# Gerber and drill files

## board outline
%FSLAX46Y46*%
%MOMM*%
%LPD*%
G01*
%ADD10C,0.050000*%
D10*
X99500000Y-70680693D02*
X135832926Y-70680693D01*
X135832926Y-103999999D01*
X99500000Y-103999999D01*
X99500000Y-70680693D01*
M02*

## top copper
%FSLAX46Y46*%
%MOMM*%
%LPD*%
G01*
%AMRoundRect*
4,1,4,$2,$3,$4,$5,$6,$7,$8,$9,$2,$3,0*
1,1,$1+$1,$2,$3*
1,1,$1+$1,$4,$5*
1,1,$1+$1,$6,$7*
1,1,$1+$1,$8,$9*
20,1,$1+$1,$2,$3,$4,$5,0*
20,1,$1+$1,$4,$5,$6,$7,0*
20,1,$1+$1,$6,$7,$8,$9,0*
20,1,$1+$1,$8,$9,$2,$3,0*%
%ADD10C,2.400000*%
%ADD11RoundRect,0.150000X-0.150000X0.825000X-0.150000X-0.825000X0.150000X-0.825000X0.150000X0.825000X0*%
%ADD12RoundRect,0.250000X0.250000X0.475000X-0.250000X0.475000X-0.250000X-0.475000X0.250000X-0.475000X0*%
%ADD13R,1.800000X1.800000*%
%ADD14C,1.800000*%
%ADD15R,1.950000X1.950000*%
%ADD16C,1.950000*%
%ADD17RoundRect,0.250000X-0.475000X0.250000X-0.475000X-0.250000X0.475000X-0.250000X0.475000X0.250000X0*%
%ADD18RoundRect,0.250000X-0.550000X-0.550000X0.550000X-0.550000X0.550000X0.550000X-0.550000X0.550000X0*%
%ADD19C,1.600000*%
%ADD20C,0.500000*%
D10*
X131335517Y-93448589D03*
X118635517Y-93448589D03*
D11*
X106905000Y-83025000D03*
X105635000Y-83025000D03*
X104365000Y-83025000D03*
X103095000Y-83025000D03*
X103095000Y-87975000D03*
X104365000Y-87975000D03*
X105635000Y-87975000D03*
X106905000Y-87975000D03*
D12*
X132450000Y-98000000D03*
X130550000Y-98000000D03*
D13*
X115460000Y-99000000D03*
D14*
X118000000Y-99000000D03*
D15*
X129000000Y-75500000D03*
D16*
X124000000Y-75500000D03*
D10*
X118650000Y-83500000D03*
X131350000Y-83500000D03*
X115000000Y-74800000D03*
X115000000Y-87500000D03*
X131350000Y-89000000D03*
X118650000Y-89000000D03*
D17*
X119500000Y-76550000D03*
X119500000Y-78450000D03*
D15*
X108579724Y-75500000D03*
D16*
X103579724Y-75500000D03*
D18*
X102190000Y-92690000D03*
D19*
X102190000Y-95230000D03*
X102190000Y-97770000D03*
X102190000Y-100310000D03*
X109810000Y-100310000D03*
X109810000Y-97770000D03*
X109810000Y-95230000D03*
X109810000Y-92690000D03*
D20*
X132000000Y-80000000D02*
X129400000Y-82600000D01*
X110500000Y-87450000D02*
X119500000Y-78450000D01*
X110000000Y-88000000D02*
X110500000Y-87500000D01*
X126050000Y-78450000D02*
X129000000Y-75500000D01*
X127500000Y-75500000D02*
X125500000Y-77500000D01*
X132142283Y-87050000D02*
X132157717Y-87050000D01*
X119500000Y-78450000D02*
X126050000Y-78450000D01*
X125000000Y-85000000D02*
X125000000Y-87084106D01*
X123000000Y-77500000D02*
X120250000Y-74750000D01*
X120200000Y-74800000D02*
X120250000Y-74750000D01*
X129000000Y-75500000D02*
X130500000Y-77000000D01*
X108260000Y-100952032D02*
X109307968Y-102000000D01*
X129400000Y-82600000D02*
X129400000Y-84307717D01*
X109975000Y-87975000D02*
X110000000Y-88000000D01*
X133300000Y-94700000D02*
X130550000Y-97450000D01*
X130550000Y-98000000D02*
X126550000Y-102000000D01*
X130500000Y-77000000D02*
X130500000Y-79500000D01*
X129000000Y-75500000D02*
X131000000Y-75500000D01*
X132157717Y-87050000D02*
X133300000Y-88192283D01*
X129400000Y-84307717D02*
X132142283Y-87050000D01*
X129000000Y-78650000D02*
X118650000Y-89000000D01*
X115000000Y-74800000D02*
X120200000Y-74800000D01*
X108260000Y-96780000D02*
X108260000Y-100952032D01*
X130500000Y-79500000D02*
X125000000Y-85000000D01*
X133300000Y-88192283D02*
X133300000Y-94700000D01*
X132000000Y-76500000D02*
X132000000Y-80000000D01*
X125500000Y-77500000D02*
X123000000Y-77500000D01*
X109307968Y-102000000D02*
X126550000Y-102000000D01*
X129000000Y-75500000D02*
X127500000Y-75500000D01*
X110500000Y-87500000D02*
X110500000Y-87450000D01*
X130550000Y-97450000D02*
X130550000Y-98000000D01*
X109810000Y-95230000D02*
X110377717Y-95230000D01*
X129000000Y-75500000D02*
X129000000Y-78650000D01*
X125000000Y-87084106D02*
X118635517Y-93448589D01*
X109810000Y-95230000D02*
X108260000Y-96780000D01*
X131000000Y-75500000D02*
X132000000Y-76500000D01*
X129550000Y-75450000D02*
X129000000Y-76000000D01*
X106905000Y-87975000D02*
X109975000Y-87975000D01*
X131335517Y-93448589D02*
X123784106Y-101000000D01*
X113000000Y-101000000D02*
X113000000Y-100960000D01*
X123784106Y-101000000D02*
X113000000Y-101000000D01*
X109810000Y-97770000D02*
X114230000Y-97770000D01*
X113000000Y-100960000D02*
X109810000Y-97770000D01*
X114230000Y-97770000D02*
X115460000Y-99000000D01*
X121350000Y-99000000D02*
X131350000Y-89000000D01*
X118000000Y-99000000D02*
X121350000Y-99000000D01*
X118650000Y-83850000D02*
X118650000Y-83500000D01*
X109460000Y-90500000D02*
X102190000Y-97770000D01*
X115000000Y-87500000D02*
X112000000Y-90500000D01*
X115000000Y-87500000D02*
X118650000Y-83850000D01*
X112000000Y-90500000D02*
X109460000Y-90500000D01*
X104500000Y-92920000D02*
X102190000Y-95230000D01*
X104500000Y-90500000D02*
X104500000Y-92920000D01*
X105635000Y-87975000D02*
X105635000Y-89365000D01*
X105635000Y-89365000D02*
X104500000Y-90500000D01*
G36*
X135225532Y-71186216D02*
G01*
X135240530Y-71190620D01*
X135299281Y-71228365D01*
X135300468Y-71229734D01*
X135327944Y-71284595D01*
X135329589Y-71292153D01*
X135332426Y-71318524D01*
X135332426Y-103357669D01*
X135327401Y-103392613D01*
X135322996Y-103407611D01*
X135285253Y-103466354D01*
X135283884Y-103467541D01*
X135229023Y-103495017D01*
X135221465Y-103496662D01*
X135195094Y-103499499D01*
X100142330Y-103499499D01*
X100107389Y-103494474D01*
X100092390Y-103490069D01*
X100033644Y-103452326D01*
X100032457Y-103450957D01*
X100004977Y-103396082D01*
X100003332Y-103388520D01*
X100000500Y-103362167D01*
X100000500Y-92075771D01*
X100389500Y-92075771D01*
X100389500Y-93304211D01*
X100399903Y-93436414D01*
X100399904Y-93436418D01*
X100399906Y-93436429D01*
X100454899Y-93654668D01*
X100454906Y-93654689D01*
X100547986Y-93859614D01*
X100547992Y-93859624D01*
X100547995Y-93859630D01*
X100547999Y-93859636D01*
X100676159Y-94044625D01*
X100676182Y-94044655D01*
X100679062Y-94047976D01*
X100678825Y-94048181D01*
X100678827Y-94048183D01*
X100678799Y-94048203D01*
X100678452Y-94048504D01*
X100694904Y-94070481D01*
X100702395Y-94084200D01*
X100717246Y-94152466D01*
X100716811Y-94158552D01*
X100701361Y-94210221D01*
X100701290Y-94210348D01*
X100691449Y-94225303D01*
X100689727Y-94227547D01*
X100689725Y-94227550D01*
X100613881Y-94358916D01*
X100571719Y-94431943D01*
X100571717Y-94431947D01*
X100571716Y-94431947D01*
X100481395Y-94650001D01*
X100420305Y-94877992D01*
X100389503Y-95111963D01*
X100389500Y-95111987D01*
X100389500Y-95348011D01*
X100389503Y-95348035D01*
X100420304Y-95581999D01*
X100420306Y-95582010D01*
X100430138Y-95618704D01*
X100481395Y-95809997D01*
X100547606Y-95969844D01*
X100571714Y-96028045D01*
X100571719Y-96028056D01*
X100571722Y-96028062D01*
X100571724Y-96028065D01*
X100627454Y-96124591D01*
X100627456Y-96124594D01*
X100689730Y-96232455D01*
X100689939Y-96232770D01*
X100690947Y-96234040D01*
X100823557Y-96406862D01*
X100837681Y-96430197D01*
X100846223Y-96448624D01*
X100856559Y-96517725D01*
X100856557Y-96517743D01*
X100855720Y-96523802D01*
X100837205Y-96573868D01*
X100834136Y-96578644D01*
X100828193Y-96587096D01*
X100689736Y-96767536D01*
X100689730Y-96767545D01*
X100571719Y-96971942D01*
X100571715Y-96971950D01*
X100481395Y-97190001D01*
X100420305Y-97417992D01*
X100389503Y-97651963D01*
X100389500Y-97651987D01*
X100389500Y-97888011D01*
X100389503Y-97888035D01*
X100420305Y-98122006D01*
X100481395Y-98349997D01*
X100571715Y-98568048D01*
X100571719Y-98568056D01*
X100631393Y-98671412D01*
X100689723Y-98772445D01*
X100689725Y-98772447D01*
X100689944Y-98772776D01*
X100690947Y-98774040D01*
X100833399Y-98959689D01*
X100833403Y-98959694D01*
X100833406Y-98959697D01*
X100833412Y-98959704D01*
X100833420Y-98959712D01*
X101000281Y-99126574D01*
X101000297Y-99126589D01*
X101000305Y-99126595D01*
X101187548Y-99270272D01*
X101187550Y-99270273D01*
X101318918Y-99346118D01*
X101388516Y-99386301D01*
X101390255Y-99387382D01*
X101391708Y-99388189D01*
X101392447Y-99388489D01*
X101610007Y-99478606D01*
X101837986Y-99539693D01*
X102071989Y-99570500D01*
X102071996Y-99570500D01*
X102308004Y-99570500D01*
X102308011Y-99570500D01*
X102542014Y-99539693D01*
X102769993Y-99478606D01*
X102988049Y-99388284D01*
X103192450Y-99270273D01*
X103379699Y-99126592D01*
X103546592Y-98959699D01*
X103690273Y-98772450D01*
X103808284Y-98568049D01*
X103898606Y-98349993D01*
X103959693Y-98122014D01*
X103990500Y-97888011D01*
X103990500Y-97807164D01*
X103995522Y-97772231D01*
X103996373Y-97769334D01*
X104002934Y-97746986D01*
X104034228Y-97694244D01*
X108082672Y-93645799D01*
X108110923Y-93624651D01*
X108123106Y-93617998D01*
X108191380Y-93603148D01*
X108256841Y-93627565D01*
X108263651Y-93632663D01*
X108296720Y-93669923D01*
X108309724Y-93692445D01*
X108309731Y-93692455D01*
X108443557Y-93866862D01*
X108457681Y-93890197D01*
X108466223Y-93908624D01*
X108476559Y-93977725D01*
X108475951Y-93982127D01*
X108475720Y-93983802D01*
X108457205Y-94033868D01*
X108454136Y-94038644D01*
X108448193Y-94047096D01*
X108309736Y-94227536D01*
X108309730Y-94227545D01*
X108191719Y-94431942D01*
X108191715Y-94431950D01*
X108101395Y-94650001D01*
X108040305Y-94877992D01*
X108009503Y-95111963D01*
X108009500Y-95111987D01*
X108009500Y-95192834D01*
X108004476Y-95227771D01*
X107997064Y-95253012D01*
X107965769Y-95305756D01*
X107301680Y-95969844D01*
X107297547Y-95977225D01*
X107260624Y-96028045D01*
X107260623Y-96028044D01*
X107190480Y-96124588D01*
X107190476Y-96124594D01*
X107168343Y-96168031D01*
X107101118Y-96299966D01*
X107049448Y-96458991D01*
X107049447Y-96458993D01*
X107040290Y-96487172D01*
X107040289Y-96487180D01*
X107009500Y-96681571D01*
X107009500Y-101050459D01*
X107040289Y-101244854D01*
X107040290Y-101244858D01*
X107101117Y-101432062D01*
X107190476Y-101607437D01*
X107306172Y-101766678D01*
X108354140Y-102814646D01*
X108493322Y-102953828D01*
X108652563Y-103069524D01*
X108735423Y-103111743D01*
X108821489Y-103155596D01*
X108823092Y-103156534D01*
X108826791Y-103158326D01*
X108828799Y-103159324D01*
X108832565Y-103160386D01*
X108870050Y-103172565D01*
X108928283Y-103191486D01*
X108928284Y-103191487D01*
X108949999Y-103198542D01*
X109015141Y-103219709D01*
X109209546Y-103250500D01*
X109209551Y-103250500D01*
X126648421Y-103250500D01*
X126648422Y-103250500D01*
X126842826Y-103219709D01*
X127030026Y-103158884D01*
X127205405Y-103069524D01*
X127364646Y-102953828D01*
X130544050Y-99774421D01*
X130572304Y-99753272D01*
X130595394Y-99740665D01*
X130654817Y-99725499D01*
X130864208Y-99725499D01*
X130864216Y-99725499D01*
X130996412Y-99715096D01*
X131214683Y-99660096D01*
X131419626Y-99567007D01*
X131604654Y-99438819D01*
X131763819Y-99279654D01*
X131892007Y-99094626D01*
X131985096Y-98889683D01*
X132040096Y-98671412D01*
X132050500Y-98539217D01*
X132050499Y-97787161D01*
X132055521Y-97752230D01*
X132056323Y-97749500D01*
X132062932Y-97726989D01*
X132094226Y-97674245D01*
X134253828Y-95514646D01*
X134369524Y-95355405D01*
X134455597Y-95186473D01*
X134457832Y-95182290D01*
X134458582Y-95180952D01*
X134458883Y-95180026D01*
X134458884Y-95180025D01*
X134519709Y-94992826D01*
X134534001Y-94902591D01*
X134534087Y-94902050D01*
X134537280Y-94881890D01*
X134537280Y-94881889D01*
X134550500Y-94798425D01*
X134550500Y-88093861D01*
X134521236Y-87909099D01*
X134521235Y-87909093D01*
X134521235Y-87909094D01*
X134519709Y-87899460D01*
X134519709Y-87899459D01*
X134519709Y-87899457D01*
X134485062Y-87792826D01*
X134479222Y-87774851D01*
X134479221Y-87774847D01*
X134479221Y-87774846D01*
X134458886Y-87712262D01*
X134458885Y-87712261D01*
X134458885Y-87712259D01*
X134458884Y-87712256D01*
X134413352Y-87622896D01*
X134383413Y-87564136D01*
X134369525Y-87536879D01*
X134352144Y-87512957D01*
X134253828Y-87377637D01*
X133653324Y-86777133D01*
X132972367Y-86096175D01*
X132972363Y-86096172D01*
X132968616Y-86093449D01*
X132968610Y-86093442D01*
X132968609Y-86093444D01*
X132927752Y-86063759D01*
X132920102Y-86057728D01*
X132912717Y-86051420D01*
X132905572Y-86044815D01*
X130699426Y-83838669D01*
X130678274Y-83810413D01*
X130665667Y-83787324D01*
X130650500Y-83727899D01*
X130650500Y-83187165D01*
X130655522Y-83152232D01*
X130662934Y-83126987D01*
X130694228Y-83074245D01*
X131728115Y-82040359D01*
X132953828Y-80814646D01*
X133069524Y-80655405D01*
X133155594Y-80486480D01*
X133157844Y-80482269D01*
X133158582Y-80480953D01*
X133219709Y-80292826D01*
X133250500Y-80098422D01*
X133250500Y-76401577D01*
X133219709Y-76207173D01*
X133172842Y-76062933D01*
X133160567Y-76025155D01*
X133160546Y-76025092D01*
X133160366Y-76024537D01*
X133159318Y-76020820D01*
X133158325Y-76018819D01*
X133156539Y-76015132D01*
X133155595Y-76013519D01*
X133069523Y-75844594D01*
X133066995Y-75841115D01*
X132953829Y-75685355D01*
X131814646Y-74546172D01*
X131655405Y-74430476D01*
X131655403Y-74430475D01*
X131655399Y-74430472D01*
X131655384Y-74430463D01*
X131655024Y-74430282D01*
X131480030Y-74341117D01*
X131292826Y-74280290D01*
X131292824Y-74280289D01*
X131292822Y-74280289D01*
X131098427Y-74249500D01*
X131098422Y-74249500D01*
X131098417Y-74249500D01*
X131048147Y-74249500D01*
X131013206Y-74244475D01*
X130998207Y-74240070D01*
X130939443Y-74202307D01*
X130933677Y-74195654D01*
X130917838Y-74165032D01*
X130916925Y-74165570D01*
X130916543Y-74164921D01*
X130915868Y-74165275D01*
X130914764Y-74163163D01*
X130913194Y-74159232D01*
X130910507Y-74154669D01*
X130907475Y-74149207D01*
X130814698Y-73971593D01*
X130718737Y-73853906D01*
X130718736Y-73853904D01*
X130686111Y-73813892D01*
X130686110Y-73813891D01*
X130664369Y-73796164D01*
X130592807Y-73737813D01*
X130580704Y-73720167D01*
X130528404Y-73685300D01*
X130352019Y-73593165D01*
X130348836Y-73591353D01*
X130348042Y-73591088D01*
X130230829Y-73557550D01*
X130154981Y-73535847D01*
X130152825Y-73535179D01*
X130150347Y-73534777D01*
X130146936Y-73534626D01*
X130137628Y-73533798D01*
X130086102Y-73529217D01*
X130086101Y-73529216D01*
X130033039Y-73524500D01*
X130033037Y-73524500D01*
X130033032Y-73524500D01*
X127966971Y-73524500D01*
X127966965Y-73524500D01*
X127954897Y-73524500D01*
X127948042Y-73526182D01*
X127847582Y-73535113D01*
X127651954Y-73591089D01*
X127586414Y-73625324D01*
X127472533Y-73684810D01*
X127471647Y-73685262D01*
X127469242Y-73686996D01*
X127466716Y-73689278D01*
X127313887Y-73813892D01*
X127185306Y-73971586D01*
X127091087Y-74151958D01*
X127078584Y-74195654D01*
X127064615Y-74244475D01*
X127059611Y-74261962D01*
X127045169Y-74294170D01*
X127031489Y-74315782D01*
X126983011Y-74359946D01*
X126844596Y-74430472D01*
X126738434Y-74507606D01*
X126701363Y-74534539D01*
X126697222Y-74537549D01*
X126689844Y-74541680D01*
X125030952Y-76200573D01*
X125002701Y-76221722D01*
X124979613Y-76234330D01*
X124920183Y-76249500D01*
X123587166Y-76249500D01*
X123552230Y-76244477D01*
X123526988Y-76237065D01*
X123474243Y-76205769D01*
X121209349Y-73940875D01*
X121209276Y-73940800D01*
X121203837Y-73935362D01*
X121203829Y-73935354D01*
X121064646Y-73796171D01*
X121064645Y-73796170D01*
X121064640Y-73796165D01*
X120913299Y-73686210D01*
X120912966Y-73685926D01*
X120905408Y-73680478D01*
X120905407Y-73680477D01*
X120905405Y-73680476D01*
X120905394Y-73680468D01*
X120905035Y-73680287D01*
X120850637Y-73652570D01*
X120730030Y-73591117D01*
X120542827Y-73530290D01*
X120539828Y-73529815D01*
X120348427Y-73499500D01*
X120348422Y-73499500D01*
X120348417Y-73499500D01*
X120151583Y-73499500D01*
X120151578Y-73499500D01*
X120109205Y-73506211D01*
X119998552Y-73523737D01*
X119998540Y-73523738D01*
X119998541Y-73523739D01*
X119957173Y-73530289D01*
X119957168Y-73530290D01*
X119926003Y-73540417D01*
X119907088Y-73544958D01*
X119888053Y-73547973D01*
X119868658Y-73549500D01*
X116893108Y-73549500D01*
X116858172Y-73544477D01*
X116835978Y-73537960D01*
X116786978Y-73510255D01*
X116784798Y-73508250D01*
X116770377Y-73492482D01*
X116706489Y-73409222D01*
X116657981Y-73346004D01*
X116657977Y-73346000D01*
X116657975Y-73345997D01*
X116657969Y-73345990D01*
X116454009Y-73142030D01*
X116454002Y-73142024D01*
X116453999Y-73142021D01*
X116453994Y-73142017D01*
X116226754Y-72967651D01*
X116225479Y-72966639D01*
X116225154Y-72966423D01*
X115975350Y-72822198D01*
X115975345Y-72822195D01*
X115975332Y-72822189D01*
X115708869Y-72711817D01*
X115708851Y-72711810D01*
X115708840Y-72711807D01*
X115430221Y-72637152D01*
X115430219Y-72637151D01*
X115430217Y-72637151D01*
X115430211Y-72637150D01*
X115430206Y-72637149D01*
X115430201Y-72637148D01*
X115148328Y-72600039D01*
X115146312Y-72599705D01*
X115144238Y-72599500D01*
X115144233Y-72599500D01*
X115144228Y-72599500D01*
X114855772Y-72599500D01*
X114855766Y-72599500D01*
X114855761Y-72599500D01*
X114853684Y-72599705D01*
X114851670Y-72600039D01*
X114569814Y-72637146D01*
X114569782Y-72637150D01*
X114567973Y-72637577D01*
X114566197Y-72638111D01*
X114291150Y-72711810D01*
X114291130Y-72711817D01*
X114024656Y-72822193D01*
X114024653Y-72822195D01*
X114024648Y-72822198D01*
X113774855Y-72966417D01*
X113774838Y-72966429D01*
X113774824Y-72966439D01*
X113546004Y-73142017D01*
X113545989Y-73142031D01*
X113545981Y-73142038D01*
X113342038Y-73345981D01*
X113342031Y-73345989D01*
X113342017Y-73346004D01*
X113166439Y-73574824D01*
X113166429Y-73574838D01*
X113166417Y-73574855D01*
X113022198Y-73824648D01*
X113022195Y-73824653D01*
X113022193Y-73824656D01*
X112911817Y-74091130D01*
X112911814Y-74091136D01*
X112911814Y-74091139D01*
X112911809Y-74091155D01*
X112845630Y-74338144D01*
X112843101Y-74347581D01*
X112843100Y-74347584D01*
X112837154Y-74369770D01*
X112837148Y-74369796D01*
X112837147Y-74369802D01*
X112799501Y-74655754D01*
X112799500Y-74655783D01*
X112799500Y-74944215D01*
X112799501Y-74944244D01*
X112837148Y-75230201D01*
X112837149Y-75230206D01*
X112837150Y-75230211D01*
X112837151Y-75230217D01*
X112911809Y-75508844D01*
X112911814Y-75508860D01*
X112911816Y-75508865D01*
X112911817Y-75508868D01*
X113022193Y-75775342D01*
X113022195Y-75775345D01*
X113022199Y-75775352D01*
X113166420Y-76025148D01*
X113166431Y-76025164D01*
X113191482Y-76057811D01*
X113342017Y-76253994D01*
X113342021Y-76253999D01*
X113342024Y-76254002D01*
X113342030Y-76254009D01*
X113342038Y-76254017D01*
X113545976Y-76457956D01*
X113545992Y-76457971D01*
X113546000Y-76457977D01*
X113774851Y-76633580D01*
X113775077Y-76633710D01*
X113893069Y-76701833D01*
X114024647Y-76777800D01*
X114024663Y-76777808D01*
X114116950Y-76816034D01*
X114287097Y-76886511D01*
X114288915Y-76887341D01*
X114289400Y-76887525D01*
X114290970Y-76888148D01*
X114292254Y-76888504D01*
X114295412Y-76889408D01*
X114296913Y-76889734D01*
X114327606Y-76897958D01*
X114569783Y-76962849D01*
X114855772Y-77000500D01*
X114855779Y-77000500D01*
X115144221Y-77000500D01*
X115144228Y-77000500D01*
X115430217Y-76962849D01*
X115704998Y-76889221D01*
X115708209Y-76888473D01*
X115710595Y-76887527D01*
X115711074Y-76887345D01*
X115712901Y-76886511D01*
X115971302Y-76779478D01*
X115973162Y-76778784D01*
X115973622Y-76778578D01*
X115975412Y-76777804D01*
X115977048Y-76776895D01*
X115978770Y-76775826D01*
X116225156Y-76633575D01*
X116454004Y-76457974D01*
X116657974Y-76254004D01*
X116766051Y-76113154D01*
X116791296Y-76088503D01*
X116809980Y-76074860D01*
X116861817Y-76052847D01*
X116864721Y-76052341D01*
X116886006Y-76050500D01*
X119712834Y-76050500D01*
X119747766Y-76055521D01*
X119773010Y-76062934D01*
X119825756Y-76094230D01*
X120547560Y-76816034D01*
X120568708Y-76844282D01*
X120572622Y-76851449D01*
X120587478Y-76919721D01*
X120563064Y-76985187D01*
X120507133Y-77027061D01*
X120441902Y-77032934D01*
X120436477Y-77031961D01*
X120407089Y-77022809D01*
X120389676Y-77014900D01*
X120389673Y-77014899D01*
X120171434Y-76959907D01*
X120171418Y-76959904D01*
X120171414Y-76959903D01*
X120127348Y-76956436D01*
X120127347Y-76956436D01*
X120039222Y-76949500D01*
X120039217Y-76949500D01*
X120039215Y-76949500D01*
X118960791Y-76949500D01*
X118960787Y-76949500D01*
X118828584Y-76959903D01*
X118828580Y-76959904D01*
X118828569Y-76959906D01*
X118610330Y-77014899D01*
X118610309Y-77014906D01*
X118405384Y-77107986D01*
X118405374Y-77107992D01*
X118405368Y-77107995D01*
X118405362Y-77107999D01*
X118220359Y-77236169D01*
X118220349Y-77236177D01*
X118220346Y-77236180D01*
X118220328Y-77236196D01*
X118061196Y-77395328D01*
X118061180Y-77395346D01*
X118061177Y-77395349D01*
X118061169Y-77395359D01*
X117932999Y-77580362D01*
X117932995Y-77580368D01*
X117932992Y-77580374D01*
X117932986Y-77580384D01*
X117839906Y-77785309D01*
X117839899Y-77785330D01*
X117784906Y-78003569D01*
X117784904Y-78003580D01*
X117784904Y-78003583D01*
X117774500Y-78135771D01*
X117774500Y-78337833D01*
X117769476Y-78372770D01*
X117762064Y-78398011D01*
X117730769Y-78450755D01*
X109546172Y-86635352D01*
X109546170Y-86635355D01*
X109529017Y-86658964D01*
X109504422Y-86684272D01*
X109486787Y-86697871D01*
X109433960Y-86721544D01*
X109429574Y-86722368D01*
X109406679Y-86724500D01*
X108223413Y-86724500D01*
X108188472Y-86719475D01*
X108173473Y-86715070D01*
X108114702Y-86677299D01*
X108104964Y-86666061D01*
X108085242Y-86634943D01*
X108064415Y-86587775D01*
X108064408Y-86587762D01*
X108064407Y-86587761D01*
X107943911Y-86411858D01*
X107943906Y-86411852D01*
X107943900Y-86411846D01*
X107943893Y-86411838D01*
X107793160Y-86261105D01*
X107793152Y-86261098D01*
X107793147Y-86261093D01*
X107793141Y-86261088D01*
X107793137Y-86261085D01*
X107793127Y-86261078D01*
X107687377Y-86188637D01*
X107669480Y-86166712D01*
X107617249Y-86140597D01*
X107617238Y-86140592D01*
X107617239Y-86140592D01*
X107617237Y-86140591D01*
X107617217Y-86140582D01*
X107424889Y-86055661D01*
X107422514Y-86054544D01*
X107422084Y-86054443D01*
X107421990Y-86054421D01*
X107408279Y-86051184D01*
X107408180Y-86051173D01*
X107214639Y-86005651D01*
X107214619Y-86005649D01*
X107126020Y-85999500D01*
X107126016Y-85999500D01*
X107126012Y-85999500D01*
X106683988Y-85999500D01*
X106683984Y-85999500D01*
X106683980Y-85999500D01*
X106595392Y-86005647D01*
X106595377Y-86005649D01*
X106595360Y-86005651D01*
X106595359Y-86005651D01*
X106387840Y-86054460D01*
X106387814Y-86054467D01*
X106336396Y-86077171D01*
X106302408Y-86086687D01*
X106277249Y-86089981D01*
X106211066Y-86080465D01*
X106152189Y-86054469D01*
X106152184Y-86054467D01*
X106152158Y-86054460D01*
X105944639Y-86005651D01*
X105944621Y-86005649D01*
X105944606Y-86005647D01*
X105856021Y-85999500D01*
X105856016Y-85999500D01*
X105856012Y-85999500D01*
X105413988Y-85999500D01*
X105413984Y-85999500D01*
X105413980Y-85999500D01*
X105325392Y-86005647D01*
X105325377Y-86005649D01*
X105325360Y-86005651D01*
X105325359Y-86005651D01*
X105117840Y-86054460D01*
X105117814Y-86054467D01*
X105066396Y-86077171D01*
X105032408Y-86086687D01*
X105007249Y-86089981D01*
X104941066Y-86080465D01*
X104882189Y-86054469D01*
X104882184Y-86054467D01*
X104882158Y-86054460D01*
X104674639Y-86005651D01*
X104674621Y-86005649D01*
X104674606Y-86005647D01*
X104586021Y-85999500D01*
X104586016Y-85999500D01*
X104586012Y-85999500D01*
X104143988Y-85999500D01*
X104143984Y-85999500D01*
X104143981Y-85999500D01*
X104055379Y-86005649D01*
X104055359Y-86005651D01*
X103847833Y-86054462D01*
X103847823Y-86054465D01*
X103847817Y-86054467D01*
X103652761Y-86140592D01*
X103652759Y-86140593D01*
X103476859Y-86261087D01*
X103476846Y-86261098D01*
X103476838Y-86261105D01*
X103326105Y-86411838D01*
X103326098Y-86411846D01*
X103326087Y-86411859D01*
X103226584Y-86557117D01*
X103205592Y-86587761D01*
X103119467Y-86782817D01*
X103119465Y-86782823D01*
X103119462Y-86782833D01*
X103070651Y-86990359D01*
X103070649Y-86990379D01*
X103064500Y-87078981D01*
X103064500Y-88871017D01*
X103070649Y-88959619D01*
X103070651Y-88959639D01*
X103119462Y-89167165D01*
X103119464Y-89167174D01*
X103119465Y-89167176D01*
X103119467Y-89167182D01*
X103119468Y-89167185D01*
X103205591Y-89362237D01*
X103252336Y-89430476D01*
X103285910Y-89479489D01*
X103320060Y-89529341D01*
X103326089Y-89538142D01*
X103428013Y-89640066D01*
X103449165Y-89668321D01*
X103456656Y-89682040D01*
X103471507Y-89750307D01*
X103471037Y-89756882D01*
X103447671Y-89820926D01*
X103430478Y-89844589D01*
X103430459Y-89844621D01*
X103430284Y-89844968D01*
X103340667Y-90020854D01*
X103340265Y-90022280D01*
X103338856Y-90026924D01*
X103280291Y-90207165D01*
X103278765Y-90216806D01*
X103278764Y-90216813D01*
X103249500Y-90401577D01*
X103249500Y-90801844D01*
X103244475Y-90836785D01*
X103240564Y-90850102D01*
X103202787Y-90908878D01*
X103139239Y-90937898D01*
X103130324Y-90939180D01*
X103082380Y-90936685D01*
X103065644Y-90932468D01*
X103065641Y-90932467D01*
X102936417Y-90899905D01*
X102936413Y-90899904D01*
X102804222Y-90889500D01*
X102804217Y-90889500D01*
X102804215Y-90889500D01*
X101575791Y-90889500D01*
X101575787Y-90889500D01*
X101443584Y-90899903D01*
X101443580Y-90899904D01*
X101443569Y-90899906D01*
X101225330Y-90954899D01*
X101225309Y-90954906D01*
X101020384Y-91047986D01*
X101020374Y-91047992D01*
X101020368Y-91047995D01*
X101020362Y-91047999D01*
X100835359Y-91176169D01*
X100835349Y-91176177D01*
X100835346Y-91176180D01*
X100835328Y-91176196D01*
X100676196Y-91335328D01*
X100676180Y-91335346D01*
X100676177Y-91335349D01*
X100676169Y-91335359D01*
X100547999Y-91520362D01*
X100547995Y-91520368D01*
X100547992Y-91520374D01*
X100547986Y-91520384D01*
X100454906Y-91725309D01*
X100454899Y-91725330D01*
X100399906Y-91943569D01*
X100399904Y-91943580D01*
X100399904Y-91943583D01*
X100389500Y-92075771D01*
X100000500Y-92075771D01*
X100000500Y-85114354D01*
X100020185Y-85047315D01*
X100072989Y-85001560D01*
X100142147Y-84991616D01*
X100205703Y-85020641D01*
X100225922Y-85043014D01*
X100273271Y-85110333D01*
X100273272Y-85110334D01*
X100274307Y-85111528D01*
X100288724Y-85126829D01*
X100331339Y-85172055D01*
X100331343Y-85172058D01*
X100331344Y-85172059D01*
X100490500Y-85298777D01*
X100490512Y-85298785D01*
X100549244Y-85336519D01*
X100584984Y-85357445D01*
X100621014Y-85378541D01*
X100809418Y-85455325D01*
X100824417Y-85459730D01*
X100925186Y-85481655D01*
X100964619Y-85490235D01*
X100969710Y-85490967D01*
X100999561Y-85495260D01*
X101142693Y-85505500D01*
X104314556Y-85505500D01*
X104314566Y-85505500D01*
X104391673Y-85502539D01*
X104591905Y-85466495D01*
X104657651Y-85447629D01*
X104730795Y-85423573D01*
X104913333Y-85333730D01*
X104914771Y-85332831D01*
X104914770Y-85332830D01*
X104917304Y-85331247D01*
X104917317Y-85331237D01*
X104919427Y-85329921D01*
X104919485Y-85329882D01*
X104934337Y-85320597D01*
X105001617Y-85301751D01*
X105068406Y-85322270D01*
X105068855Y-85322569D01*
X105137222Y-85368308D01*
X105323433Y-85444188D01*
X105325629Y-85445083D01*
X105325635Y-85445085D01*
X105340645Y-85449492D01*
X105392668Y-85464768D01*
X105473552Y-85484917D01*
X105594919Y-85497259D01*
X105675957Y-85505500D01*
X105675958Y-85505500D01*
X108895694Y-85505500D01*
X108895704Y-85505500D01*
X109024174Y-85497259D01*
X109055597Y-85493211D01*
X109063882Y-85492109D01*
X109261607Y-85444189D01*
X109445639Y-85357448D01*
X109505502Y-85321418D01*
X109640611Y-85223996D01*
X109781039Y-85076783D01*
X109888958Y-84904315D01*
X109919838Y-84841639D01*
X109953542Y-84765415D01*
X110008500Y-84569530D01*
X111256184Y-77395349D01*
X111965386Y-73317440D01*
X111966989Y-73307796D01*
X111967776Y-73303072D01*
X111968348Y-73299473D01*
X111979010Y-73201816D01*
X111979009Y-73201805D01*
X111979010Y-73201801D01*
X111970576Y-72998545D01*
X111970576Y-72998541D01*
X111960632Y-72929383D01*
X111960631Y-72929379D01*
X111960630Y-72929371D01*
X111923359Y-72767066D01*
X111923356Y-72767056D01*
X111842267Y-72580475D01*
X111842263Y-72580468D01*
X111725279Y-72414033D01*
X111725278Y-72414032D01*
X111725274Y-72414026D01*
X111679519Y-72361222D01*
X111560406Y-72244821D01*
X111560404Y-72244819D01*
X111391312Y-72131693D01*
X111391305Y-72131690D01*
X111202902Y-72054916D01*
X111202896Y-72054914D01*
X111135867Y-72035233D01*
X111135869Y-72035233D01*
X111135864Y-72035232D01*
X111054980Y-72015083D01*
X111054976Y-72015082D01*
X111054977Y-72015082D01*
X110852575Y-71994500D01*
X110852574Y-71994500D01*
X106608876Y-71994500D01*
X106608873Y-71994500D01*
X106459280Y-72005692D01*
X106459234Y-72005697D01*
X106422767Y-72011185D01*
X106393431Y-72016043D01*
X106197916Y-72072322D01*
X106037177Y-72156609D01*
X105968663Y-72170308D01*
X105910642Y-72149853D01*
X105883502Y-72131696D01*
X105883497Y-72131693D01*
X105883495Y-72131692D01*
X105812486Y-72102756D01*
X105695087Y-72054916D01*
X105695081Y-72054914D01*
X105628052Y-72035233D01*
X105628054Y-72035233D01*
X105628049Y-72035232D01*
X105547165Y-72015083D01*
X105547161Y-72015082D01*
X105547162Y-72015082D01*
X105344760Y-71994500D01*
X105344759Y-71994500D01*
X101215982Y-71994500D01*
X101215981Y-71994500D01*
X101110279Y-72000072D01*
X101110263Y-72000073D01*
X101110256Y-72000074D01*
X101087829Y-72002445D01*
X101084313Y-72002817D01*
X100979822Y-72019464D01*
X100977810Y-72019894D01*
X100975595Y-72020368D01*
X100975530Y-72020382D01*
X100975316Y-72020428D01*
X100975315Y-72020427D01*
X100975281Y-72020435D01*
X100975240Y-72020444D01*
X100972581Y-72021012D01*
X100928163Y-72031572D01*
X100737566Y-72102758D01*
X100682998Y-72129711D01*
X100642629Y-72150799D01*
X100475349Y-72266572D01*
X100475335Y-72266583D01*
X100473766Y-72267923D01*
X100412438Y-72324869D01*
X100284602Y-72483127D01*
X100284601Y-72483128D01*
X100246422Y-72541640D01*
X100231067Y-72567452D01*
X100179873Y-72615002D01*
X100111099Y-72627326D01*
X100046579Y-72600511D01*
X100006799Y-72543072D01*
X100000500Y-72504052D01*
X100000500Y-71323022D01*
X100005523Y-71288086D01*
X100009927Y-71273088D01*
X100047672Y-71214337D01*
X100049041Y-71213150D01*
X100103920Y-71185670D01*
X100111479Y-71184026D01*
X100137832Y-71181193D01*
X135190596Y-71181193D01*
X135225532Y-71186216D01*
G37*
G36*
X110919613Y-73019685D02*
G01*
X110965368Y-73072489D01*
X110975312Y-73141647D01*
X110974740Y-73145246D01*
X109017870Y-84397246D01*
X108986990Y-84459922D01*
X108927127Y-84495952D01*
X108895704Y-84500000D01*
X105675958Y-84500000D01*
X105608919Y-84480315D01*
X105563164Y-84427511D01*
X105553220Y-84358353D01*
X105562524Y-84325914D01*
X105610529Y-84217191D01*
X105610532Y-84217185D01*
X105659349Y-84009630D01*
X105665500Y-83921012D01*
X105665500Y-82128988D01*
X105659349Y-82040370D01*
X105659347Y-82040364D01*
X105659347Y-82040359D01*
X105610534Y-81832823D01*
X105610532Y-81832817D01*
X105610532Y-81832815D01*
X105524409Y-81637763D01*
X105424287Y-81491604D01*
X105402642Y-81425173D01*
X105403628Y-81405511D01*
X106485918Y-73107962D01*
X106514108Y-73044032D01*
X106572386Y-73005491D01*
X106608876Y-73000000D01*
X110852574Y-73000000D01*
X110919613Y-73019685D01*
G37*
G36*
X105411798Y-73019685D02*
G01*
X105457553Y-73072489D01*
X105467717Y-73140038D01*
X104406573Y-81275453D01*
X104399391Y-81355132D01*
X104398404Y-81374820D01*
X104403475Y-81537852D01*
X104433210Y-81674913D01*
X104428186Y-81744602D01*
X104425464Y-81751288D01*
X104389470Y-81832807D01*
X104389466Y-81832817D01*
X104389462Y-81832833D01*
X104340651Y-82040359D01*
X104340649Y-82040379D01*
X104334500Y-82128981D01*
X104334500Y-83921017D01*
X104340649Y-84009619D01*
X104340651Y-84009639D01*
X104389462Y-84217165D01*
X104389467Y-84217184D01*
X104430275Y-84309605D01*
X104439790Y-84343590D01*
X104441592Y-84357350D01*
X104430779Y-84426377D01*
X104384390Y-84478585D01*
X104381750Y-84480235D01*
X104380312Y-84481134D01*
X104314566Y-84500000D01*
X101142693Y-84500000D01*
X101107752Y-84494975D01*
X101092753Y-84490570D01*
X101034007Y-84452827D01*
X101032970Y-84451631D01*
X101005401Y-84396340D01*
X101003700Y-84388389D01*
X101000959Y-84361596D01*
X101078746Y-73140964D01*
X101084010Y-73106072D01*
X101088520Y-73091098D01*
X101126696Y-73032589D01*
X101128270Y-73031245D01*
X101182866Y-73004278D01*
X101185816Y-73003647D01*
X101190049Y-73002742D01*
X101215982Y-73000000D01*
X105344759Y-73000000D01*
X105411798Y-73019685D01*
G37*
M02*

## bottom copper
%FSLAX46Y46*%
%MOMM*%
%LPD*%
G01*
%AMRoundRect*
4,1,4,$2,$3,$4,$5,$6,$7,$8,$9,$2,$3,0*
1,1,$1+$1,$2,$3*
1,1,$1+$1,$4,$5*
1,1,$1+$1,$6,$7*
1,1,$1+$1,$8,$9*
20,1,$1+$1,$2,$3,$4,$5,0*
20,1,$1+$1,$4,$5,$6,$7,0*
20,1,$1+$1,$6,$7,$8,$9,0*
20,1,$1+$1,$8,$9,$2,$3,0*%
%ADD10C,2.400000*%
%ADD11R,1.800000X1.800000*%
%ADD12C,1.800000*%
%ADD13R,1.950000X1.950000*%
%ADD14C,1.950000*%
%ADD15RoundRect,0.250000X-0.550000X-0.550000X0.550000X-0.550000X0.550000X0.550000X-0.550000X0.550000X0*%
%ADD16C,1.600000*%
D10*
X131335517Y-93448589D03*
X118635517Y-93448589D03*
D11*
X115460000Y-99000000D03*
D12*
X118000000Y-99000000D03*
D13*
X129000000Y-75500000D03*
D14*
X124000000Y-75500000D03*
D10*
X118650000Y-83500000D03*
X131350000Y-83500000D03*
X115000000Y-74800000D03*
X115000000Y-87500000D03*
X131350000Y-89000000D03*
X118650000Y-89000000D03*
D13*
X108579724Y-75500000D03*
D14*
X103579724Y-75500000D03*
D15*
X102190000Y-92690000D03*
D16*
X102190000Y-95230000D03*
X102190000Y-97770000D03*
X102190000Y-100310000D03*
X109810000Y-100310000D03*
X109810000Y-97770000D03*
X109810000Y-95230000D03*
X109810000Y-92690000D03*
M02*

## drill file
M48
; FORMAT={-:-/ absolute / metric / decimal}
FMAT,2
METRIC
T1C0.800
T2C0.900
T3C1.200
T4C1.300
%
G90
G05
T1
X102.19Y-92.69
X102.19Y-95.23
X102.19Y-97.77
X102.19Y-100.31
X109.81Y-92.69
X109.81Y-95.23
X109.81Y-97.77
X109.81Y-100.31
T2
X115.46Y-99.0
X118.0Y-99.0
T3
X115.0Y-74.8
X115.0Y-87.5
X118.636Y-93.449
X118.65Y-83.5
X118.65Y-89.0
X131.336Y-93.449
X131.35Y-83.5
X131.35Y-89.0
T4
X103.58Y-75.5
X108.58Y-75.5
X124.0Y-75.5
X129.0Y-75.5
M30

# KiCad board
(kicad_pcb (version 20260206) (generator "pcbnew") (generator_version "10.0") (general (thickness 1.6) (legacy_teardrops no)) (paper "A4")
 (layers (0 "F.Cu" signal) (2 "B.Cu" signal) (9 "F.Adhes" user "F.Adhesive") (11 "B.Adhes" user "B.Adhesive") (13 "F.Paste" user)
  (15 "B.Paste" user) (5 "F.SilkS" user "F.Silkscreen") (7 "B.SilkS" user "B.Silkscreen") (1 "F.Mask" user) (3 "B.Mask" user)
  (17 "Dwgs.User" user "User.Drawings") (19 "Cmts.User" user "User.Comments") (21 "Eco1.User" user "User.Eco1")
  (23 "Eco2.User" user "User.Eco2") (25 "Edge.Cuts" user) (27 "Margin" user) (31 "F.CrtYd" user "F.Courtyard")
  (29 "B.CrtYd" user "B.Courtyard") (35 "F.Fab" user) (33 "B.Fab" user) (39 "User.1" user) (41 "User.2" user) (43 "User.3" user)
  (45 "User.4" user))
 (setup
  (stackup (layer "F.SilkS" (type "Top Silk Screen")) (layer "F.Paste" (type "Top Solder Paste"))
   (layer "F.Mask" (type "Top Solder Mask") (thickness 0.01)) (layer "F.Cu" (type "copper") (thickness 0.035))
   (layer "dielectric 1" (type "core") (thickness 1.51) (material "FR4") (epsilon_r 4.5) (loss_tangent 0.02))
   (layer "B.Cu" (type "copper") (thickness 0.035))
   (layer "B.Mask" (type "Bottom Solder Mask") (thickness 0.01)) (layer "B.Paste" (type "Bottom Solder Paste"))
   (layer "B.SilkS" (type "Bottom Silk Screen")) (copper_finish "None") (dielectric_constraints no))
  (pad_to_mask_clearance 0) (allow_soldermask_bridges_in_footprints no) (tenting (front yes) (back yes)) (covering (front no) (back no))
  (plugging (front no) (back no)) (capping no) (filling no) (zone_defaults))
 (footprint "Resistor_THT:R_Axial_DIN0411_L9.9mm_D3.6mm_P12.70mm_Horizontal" (layer "F.Cu") (at 131.335517 93.448589 180)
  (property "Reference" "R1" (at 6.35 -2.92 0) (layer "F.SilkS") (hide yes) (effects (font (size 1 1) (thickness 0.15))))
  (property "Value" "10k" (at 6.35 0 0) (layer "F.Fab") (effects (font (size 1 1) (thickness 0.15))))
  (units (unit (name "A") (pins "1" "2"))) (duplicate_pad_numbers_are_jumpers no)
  (pad "1" thru_hole circle (at 0 0 180) (size 2.4 2.4) (drill 1.2) (layers "*.Cu" "*.Mask") (remove_unused_layers no) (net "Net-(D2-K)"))
  (pad "2" thru_hole circle (at 12.7 0 180) (size 2.4 2.4) (drill 1.2) (layers "*.Cu" "*.Mask") (remove_unused_layers no) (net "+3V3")))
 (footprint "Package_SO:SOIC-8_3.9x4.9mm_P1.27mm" (layer "F.Cu") (at 105 85.5 -90)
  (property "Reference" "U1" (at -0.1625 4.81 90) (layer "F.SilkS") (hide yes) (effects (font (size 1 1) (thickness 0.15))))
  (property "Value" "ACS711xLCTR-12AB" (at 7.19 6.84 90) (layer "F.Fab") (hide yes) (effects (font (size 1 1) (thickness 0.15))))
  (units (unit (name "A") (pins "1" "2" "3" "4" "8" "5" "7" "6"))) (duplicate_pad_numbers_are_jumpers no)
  (pad "1" smd roundrect (at -2.475 -1.905 270) (size 1.95 0.6) (layers "F.Cu" "F.Mask" "F.Paste") (roundrect_rratio 0.25) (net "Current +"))
  (pad "2" smd roundrect (at -2.475 -0.635 270) (size 1.95 0.6) (layers "F.Cu" "F.Mask" "F.Paste") (roundrect_rratio 0.25) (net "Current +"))
  (pad "3" smd roundrect (at -2.475 0.635 270) (size 1.95 0.6) (layers "F.Cu" "F.Mask" "F.Paste") (roundrect_rratio 0.25) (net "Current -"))
  (pad "4" smd roundrect (at -2.475 1.905 270) (size 1.95 0.6) (layers "F.Cu" "F.Mask" "F.Paste") (roundrect_rratio 0.25) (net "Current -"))
  (pad "5" smd roundrect (at 2.475 1.905 270) (size 1.95 0.6) (layers "F.Cu" "F.Mask" "F.Paste") (roundrect_rratio 0.25) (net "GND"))
  (pad "6" smd roundrect (at 2.475 0.635 270) (size 1.95 0.6) (layers "F.Cu" "F.Mask" "F.Paste") (roundrect_rratio 0.25)
   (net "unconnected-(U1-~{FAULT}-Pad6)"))
  (pad "7" smd roundrect (at 2.475 -0.635 270) (size 1.95 0.6) (layers "F.Cu" "F.Mask" "F.Paste") (roundrect_rratio 0.25)
   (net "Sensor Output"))
  (pad "8" smd roundrect (at 2.475 -1.905 270) (size 1.95 0.6) (layers "F.Cu" "F.Mask" "F.Paste") (roundrect_rratio 0.25) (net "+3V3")))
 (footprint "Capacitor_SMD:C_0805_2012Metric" (layer "F.Cu") (at 131.5 98 180)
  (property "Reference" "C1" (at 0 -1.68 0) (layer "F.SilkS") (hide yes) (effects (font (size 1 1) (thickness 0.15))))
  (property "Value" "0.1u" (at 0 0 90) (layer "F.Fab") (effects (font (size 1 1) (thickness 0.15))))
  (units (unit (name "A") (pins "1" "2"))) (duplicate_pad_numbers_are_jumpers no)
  (pad "1" smd roundrect (at -0.95 0 180) (size 1 1.45) (layers "F.Cu" "F.Mask" "F.Paste") (roundrect_rratio 0.25) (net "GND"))
  (pad "2" smd roundrect (at 0.95 0 180) (size 1 1.45) (layers "F.Cu" "F.Mask" "F.Paste") (roundrect_rratio 0.25) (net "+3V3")))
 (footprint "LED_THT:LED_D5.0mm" (layer "F.Cu") (at 115.46 99)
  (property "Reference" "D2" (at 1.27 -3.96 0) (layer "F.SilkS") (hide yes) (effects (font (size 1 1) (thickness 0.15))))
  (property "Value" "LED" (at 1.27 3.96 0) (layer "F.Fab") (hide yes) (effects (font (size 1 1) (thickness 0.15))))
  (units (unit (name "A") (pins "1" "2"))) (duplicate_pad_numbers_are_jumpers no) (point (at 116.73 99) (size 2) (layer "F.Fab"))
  (pad "1" thru_hole rect (at 0 0) (size 1.8 1.8) (drill 0.9) (layers "*.Cu" "*.Mask") (remove_unused_layers no) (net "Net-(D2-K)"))
  (pad "2" thru_hole circle (at 2.54 0) (size 1.8 1.8) (drill 0.9) (layers "*.Cu" "*.Mask") (remove_unused_layers no) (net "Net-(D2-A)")))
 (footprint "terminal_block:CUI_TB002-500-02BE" (layer "F.Cu") (at 129 75.5 180)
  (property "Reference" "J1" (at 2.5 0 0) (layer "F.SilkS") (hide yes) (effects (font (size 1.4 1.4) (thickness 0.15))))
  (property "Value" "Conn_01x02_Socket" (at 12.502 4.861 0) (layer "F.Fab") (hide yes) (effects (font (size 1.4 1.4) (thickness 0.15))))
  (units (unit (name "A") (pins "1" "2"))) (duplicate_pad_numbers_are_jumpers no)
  (pad "1" thru_hole rect (at 0 0 180) (size 1.95 1.95) (drill 1.3) (layers "*.Cu" "*.Mask") (remove_unused_layers no) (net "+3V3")
   (solder_mask_margin 0.102))
  (pad "2" thru_hole circle (at 5 0 180) (size 1.95 1.95) (drill 1.3) (layers "*.Cu" "*.Mask") (remove_unused_layers no) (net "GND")
   (solder_mask_margin 0.102)))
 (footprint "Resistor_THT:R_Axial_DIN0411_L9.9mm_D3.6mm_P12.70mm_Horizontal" (layer "F.Cu") (at 118.65 83.5)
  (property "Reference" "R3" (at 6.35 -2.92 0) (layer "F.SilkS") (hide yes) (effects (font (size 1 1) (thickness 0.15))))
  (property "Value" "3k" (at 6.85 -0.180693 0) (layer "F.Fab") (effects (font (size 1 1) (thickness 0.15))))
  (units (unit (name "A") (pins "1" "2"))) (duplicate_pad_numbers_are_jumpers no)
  (pad "1" thru_hole circle (at 0 0) (size 2.4 2.4) (drill 1.2) (layers "*.Cu" "*.Mask") (remove_unused_layers no) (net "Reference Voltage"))
  (pad "2" thru_hole circle (at 12.7 0) (size 2.4 2.4) (drill 1.2) (layers "*.Cu" "*.Mask") (remove_unused_layers no) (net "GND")))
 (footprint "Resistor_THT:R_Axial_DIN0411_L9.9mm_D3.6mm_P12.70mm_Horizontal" (layer "F.Cu") (at 115 74.8 -90)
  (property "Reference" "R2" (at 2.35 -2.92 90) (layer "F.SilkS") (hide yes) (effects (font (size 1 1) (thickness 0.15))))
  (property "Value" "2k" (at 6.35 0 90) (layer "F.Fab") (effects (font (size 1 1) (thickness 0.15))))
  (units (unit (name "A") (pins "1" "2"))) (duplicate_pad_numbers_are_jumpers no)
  (pad "1" thru_hole circle (at 0 0 270) (size 2.4 2.4) (drill 1.2) (layers "*.Cu" "*.Mask") (remove_unused_layers no) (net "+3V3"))
  (pad "2" thru_hole circle (at 12.7 0 270) (size 2.4 2.4) (drill 1.2) (layers "*.Cu" "*.Mask") (remove_unused_layers no)
   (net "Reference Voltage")))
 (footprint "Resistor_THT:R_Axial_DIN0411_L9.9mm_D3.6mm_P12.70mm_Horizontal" (layer "F.Cu") (at 131.35 89 180)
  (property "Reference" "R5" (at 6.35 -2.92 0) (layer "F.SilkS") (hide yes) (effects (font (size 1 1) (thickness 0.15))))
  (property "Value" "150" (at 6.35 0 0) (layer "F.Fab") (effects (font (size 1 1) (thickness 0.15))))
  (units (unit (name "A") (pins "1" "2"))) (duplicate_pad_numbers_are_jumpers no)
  (pad "1" thru_hole circle (at 0 0 180) (size 2.4 2.4) (drill 1.2) (layers "*.Cu" "*.Mask") (remove_unused_layers no) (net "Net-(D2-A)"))
  (pad "2" thru_hole circle (at 12.7 0 180) (size 2.4 2.4) (drill 1.2) (layers "*.Cu" "*.Mask") (remove_unused_layers no) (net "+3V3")))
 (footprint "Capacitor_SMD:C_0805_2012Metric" (layer "F.Cu") (at 119.5 77.5 -90)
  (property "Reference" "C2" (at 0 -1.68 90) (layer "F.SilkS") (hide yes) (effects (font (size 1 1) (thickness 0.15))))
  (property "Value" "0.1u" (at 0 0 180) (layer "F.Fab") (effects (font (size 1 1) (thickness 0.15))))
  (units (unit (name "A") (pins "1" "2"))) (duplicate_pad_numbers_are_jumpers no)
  (pad "1" smd roundrect (at -0.95 0 270) (size 1 1.45) (layers "F.Cu" "F.Mask" "F.Paste") (roundrect_rratio 0.25) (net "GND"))
  (pad "2" smd roundrect (at 0.95 0 270) (size 1 1.45) (layers "F.Cu" "F.Mask" "F.Paste") (roundrect_rratio 0.25) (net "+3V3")))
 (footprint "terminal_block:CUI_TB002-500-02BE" (layer "F.Cu") (at 108.579724 75.5 180)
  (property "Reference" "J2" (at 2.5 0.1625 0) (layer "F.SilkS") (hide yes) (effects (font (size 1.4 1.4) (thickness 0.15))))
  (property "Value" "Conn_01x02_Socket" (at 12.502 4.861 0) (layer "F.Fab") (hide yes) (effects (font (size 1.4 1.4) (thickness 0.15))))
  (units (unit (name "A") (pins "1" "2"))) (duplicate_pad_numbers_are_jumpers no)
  (pad "1" thru_hole rect (at 0 0 180) (size 1.95 1.95) (drill 1.3) (layers "*.Cu" "*.Mask") (remove_unused_layers no) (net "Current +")
   (solder_mask_margin 0.102))
  (pad "2" thru_hole circle (at 5 0 180) (size 1.95 1.95) (drill 1.3) (layers "*.Cu" "*.Mask") (remove_unused_layers no) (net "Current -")
   (solder_mask_margin 0.102)))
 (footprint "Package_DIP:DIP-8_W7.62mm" (layer "F.Cu") (at 102.19 92.69)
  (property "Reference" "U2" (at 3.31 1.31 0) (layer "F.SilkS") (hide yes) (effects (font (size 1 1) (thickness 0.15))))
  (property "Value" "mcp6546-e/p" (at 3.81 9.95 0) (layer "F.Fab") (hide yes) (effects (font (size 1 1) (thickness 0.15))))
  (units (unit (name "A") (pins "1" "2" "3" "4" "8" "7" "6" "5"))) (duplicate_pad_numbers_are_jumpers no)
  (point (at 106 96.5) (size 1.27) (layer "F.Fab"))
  (pad "1" thru_hole roundrect (at 0 0) (size 1.6 1.6) (drill 0.8) (layers "*.Cu" "*.Mask") (remove_unused_layers no)
   (roundrect_rratio 0.15625) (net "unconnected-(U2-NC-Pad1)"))
  (pad "2" thru_hole circle (at 0 2.54) (size 1.6 1.6) (drill 0.8) (layers "*.Cu" "*.Mask") (remove_unused_layers no) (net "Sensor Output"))
  (pad "3" thru_hole circle (at 0 5.08) (size 1.6 1.6) (drill 0.8) (layers "*.Cu" "*.Mask") (remove_unused_layers no)
   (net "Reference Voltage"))
  (pad "4" thru_hole circle (at 0 7.62) (size 1.6 1.6) (drill 0.8) (layers "*.Cu" "*.Mask") (remove_unused_layers no) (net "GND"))
  (pad "5" thru_hole circle (at 7.62 7.62) (size 1.6 1.6) (drill 0.8) (layers "*.Cu" "*.Mask") (remove_unused_layers no)
   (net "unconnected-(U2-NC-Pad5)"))
  (pad "6" thru_hole circle (at 7.62 5.08) (size 1.6 1.6) (drill 0.8) (layers "*.Cu" "*.Mask") (remove_unused_layers no) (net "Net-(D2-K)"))
  (pad "7" thru_hole circle (at 7.62 2.54) (size 1.6 1.6) (drill 0.8) (layers "*.Cu" "*.Mask") (remove_unused_layers no) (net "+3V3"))
  (pad "8" thru_hole circle (at 7.62 0) (size 1.6 1.6) (drill 0.8) (layers "*.Cu" "*.Mask") (remove_unused_layers no)
   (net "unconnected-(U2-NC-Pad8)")))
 (gr_rect (start 99.5 70.680693) (end 135.832926 103.999999) (stroke (width 0.05) (type default)) (fill no) (layer "Edge.Cuts"))
 (segment (start 132 80) (end 129.4 82.6) (width 0.5) (layer "F.Cu") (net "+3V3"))
 (segment (start 110.5 87.45) (end 119.5 78.45) (width 0.5) (layer "F.Cu") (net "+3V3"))
 (segment (start 110 88) (end 110.5 87.5) (width 0.5) (layer "F.Cu") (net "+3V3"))
 (segment (start 126.05 78.45) (end 129 75.5) (width 0.5) (layer "F.Cu") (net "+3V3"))
 (segment (start 127.5 75.5) (end 125.5 77.5) (width 0.5) (layer "F.Cu") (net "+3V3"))
 (segment (start 132.142283 87.05) (end 132.157717 87.05) (width 0.5) (layer "F.Cu") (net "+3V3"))
 (segment (start 119.5 78.45) (end 126.05 78.45) (width 0.5) (layer "F.Cu") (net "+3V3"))
 (segment (start 125 85) (end 125 87.084106) (width 0.5) (layer "F.Cu") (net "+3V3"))
 (segment (start 123 77.5) (end 120.25 74.75) (width 0.5) (layer "F.Cu") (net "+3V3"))
 (segment (start 120.2 74.8) (end 120.25 74.75) (width 0.5) (layer "F.Cu") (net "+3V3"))
 (segment (start 129 75.5) (end 130.5 77) (width 0.5) (layer "F.Cu") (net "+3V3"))
 (segment (start 108.26 100.952032) (end 109.307968 102) (width 0.5) (layer "F.Cu") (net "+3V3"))
 (segment (start 129.4 82.6) (end 129.4 84.307717) (width 0.5) (layer "F.Cu") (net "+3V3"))
 (segment (start 109.975 87.975) (end 110 88) (width 0.5) (layer "F.Cu") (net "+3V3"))
 (segment (start 133.3 94.7) (end 130.55 97.45) (width 0.5) (layer "F.Cu") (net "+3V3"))
 (segment (start 130.55 98) (end 126.55 102) (width 0.5) (layer "F.Cu") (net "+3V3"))
 (segment (start 130.5 77) (end 130.5 79.5) (width 0.5) (layer "F.Cu") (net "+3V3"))
 (segment (start 129 75.5) (end 131 75.5) (width 0.5) (layer "F.Cu") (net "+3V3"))
 (segment (start 132.157717 87.05) (end 133.3 88.192283) (width 0.5) (layer "F.Cu") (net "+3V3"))
 (segment (start 129.4 84.307717) (end 132.142283 87.05) (width 0.5) (layer "F.Cu") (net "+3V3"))
 (segment (start 129 78.65) (end 118.65 89) (width 0.5) (layer "F.Cu") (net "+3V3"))
 (segment (start 115 74.8) (end 120.2 74.8) (width 0.5) (layer "F.Cu") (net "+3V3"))
 (segment (start 108.26 96.78) (end 108.26 100.952032) (width 0.5) (layer "F.Cu") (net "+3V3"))
 (segment (start 130.5 79.5) (end 125 85) (width 0.5) (layer "F.Cu") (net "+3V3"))
 (segment (start 133.3 88.192283) (end 133.3 94.7) (width 0.5) (layer "F.Cu") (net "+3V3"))
 (segment (start 132 76.5) (end 132 80) (width 0.5) (layer "F.Cu") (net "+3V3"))
 (segment (start 125.5 77.5) (end 123 77.5) (width 0.5) (layer "F.Cu") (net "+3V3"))
 (segment (start 109.307968 102) (end 126.55 102) (width 0.5) (layer "F.Cu") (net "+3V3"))
 (segment (start 129 75.5) (end 127.5 75.5) (width 0.5) (layer "F.Cu") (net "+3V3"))
 (segment (start 110.5 87.5) (end 110.5 87.45) (width 0.5) (layer "F.Cu") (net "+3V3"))
 (segment (start 130.55 97.45) (end 130.55 98) (width 0.5) (layer "F.Cu") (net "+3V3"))
 (segment (start 109.81 95.23) (end 110.377717 95.23) (width 0.5) (layer "F.Cu") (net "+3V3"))
 (segment (start 129 75.5) (end 129 78.65) (width 0.5) (layer "F.Cu") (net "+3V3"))
 (segment (start 125 87.084106) (end 118.635517 93.448589) (width 0.5) (layer "F.Cu") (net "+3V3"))
 (segment (start 109.81 95.23) (end 108.26 96.78) (width 0.5) (layer "F.Cu") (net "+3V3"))
 (segment (start 131 75.5) (end 132 76.5) (width 0.5) (layer "F.Cu") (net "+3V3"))
 (segment (start 129.55 75.45) (end 129 76) (width 0.5) (layer "F.Cu") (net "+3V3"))
 (segment (start 106.905 87.975) (end 109.975 87.975) (width 0.5) (layer "F.Cu") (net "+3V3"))
 (segment (start 131.335517 93.448589) (end 123.784106 101) (width 0.5) (layer "F.Cu") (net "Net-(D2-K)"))
 (segment (start 113 101) (end 113 100.96) (width 0.5) (layer "F.Cu") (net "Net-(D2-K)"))
 (segment (start 123.784106 101) (end 113 101) (width 0.5) (layer "F.Cu") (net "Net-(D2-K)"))
 (segment (start 109.81 97.77) (end 114.23 97.77) (width 0.5) (layer "F.Cu") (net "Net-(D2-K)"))
 (segment (start 113 100.96) (end 109.81 97.77) (width 0.5) (layer "F.Cu") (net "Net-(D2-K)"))
 (segment (start 114.23 97.77) (end 115.46 99) (width 0.5) (layer "F.Cu") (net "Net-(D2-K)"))
 (segment (start 121.35 99) (end 131.35 89) (width 0.5) (layer "F.Cu") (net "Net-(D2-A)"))
 (segment (start 118 99) (end 121.35 99) (width 0.5) (layer "F.Cu") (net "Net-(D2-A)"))
 (segment (start 118.65 83.85) (end 118.65 83.5) (width 0.5) (layer "F.Cu") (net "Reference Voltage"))
 (segment (start 109.46 90.5) (end 102.19 97.77) (width 0.5) (layer "F.Cu") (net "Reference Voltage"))
 (segment (start 115 87.5) (end 112 90.5) (width 0.5) (layer "F.Cu") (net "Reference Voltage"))
 (segment (start 115 87.5) (end 118.65 83.85) (width 0.5) (layer "F.Cu") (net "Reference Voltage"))
 (segment (start 112 90.5) (end 109.46 90.5) (width 0.5) (layer "F.Cu") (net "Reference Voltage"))
 (segment (start 104.5 92.92) (end 102.19 95.23) (width 0.5) (layer "F.Cu") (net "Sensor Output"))
 (segment (start 104.5 90.5) (end 104.5 92.92) (width 0.5) (layer "F.Cu") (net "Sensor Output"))
 (segment (start 105.635 87.975) (end 105.635 89.365) (width 0.5) (layer "F.Cu") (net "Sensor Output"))
 (segment (start 105.635 89.365) (end 104.5 90.5) (width 0.5) (layer "F.Cu") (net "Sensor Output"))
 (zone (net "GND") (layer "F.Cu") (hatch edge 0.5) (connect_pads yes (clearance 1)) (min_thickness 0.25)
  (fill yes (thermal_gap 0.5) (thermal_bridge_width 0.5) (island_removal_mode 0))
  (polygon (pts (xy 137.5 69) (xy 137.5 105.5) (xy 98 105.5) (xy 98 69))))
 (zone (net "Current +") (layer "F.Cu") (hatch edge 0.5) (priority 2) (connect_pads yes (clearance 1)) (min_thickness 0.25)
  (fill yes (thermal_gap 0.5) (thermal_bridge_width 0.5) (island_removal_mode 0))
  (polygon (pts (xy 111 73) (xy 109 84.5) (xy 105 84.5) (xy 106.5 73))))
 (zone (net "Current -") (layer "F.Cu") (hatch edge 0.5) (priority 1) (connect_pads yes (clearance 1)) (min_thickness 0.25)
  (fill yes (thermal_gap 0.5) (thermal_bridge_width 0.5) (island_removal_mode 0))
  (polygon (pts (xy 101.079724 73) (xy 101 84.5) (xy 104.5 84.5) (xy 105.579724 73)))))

